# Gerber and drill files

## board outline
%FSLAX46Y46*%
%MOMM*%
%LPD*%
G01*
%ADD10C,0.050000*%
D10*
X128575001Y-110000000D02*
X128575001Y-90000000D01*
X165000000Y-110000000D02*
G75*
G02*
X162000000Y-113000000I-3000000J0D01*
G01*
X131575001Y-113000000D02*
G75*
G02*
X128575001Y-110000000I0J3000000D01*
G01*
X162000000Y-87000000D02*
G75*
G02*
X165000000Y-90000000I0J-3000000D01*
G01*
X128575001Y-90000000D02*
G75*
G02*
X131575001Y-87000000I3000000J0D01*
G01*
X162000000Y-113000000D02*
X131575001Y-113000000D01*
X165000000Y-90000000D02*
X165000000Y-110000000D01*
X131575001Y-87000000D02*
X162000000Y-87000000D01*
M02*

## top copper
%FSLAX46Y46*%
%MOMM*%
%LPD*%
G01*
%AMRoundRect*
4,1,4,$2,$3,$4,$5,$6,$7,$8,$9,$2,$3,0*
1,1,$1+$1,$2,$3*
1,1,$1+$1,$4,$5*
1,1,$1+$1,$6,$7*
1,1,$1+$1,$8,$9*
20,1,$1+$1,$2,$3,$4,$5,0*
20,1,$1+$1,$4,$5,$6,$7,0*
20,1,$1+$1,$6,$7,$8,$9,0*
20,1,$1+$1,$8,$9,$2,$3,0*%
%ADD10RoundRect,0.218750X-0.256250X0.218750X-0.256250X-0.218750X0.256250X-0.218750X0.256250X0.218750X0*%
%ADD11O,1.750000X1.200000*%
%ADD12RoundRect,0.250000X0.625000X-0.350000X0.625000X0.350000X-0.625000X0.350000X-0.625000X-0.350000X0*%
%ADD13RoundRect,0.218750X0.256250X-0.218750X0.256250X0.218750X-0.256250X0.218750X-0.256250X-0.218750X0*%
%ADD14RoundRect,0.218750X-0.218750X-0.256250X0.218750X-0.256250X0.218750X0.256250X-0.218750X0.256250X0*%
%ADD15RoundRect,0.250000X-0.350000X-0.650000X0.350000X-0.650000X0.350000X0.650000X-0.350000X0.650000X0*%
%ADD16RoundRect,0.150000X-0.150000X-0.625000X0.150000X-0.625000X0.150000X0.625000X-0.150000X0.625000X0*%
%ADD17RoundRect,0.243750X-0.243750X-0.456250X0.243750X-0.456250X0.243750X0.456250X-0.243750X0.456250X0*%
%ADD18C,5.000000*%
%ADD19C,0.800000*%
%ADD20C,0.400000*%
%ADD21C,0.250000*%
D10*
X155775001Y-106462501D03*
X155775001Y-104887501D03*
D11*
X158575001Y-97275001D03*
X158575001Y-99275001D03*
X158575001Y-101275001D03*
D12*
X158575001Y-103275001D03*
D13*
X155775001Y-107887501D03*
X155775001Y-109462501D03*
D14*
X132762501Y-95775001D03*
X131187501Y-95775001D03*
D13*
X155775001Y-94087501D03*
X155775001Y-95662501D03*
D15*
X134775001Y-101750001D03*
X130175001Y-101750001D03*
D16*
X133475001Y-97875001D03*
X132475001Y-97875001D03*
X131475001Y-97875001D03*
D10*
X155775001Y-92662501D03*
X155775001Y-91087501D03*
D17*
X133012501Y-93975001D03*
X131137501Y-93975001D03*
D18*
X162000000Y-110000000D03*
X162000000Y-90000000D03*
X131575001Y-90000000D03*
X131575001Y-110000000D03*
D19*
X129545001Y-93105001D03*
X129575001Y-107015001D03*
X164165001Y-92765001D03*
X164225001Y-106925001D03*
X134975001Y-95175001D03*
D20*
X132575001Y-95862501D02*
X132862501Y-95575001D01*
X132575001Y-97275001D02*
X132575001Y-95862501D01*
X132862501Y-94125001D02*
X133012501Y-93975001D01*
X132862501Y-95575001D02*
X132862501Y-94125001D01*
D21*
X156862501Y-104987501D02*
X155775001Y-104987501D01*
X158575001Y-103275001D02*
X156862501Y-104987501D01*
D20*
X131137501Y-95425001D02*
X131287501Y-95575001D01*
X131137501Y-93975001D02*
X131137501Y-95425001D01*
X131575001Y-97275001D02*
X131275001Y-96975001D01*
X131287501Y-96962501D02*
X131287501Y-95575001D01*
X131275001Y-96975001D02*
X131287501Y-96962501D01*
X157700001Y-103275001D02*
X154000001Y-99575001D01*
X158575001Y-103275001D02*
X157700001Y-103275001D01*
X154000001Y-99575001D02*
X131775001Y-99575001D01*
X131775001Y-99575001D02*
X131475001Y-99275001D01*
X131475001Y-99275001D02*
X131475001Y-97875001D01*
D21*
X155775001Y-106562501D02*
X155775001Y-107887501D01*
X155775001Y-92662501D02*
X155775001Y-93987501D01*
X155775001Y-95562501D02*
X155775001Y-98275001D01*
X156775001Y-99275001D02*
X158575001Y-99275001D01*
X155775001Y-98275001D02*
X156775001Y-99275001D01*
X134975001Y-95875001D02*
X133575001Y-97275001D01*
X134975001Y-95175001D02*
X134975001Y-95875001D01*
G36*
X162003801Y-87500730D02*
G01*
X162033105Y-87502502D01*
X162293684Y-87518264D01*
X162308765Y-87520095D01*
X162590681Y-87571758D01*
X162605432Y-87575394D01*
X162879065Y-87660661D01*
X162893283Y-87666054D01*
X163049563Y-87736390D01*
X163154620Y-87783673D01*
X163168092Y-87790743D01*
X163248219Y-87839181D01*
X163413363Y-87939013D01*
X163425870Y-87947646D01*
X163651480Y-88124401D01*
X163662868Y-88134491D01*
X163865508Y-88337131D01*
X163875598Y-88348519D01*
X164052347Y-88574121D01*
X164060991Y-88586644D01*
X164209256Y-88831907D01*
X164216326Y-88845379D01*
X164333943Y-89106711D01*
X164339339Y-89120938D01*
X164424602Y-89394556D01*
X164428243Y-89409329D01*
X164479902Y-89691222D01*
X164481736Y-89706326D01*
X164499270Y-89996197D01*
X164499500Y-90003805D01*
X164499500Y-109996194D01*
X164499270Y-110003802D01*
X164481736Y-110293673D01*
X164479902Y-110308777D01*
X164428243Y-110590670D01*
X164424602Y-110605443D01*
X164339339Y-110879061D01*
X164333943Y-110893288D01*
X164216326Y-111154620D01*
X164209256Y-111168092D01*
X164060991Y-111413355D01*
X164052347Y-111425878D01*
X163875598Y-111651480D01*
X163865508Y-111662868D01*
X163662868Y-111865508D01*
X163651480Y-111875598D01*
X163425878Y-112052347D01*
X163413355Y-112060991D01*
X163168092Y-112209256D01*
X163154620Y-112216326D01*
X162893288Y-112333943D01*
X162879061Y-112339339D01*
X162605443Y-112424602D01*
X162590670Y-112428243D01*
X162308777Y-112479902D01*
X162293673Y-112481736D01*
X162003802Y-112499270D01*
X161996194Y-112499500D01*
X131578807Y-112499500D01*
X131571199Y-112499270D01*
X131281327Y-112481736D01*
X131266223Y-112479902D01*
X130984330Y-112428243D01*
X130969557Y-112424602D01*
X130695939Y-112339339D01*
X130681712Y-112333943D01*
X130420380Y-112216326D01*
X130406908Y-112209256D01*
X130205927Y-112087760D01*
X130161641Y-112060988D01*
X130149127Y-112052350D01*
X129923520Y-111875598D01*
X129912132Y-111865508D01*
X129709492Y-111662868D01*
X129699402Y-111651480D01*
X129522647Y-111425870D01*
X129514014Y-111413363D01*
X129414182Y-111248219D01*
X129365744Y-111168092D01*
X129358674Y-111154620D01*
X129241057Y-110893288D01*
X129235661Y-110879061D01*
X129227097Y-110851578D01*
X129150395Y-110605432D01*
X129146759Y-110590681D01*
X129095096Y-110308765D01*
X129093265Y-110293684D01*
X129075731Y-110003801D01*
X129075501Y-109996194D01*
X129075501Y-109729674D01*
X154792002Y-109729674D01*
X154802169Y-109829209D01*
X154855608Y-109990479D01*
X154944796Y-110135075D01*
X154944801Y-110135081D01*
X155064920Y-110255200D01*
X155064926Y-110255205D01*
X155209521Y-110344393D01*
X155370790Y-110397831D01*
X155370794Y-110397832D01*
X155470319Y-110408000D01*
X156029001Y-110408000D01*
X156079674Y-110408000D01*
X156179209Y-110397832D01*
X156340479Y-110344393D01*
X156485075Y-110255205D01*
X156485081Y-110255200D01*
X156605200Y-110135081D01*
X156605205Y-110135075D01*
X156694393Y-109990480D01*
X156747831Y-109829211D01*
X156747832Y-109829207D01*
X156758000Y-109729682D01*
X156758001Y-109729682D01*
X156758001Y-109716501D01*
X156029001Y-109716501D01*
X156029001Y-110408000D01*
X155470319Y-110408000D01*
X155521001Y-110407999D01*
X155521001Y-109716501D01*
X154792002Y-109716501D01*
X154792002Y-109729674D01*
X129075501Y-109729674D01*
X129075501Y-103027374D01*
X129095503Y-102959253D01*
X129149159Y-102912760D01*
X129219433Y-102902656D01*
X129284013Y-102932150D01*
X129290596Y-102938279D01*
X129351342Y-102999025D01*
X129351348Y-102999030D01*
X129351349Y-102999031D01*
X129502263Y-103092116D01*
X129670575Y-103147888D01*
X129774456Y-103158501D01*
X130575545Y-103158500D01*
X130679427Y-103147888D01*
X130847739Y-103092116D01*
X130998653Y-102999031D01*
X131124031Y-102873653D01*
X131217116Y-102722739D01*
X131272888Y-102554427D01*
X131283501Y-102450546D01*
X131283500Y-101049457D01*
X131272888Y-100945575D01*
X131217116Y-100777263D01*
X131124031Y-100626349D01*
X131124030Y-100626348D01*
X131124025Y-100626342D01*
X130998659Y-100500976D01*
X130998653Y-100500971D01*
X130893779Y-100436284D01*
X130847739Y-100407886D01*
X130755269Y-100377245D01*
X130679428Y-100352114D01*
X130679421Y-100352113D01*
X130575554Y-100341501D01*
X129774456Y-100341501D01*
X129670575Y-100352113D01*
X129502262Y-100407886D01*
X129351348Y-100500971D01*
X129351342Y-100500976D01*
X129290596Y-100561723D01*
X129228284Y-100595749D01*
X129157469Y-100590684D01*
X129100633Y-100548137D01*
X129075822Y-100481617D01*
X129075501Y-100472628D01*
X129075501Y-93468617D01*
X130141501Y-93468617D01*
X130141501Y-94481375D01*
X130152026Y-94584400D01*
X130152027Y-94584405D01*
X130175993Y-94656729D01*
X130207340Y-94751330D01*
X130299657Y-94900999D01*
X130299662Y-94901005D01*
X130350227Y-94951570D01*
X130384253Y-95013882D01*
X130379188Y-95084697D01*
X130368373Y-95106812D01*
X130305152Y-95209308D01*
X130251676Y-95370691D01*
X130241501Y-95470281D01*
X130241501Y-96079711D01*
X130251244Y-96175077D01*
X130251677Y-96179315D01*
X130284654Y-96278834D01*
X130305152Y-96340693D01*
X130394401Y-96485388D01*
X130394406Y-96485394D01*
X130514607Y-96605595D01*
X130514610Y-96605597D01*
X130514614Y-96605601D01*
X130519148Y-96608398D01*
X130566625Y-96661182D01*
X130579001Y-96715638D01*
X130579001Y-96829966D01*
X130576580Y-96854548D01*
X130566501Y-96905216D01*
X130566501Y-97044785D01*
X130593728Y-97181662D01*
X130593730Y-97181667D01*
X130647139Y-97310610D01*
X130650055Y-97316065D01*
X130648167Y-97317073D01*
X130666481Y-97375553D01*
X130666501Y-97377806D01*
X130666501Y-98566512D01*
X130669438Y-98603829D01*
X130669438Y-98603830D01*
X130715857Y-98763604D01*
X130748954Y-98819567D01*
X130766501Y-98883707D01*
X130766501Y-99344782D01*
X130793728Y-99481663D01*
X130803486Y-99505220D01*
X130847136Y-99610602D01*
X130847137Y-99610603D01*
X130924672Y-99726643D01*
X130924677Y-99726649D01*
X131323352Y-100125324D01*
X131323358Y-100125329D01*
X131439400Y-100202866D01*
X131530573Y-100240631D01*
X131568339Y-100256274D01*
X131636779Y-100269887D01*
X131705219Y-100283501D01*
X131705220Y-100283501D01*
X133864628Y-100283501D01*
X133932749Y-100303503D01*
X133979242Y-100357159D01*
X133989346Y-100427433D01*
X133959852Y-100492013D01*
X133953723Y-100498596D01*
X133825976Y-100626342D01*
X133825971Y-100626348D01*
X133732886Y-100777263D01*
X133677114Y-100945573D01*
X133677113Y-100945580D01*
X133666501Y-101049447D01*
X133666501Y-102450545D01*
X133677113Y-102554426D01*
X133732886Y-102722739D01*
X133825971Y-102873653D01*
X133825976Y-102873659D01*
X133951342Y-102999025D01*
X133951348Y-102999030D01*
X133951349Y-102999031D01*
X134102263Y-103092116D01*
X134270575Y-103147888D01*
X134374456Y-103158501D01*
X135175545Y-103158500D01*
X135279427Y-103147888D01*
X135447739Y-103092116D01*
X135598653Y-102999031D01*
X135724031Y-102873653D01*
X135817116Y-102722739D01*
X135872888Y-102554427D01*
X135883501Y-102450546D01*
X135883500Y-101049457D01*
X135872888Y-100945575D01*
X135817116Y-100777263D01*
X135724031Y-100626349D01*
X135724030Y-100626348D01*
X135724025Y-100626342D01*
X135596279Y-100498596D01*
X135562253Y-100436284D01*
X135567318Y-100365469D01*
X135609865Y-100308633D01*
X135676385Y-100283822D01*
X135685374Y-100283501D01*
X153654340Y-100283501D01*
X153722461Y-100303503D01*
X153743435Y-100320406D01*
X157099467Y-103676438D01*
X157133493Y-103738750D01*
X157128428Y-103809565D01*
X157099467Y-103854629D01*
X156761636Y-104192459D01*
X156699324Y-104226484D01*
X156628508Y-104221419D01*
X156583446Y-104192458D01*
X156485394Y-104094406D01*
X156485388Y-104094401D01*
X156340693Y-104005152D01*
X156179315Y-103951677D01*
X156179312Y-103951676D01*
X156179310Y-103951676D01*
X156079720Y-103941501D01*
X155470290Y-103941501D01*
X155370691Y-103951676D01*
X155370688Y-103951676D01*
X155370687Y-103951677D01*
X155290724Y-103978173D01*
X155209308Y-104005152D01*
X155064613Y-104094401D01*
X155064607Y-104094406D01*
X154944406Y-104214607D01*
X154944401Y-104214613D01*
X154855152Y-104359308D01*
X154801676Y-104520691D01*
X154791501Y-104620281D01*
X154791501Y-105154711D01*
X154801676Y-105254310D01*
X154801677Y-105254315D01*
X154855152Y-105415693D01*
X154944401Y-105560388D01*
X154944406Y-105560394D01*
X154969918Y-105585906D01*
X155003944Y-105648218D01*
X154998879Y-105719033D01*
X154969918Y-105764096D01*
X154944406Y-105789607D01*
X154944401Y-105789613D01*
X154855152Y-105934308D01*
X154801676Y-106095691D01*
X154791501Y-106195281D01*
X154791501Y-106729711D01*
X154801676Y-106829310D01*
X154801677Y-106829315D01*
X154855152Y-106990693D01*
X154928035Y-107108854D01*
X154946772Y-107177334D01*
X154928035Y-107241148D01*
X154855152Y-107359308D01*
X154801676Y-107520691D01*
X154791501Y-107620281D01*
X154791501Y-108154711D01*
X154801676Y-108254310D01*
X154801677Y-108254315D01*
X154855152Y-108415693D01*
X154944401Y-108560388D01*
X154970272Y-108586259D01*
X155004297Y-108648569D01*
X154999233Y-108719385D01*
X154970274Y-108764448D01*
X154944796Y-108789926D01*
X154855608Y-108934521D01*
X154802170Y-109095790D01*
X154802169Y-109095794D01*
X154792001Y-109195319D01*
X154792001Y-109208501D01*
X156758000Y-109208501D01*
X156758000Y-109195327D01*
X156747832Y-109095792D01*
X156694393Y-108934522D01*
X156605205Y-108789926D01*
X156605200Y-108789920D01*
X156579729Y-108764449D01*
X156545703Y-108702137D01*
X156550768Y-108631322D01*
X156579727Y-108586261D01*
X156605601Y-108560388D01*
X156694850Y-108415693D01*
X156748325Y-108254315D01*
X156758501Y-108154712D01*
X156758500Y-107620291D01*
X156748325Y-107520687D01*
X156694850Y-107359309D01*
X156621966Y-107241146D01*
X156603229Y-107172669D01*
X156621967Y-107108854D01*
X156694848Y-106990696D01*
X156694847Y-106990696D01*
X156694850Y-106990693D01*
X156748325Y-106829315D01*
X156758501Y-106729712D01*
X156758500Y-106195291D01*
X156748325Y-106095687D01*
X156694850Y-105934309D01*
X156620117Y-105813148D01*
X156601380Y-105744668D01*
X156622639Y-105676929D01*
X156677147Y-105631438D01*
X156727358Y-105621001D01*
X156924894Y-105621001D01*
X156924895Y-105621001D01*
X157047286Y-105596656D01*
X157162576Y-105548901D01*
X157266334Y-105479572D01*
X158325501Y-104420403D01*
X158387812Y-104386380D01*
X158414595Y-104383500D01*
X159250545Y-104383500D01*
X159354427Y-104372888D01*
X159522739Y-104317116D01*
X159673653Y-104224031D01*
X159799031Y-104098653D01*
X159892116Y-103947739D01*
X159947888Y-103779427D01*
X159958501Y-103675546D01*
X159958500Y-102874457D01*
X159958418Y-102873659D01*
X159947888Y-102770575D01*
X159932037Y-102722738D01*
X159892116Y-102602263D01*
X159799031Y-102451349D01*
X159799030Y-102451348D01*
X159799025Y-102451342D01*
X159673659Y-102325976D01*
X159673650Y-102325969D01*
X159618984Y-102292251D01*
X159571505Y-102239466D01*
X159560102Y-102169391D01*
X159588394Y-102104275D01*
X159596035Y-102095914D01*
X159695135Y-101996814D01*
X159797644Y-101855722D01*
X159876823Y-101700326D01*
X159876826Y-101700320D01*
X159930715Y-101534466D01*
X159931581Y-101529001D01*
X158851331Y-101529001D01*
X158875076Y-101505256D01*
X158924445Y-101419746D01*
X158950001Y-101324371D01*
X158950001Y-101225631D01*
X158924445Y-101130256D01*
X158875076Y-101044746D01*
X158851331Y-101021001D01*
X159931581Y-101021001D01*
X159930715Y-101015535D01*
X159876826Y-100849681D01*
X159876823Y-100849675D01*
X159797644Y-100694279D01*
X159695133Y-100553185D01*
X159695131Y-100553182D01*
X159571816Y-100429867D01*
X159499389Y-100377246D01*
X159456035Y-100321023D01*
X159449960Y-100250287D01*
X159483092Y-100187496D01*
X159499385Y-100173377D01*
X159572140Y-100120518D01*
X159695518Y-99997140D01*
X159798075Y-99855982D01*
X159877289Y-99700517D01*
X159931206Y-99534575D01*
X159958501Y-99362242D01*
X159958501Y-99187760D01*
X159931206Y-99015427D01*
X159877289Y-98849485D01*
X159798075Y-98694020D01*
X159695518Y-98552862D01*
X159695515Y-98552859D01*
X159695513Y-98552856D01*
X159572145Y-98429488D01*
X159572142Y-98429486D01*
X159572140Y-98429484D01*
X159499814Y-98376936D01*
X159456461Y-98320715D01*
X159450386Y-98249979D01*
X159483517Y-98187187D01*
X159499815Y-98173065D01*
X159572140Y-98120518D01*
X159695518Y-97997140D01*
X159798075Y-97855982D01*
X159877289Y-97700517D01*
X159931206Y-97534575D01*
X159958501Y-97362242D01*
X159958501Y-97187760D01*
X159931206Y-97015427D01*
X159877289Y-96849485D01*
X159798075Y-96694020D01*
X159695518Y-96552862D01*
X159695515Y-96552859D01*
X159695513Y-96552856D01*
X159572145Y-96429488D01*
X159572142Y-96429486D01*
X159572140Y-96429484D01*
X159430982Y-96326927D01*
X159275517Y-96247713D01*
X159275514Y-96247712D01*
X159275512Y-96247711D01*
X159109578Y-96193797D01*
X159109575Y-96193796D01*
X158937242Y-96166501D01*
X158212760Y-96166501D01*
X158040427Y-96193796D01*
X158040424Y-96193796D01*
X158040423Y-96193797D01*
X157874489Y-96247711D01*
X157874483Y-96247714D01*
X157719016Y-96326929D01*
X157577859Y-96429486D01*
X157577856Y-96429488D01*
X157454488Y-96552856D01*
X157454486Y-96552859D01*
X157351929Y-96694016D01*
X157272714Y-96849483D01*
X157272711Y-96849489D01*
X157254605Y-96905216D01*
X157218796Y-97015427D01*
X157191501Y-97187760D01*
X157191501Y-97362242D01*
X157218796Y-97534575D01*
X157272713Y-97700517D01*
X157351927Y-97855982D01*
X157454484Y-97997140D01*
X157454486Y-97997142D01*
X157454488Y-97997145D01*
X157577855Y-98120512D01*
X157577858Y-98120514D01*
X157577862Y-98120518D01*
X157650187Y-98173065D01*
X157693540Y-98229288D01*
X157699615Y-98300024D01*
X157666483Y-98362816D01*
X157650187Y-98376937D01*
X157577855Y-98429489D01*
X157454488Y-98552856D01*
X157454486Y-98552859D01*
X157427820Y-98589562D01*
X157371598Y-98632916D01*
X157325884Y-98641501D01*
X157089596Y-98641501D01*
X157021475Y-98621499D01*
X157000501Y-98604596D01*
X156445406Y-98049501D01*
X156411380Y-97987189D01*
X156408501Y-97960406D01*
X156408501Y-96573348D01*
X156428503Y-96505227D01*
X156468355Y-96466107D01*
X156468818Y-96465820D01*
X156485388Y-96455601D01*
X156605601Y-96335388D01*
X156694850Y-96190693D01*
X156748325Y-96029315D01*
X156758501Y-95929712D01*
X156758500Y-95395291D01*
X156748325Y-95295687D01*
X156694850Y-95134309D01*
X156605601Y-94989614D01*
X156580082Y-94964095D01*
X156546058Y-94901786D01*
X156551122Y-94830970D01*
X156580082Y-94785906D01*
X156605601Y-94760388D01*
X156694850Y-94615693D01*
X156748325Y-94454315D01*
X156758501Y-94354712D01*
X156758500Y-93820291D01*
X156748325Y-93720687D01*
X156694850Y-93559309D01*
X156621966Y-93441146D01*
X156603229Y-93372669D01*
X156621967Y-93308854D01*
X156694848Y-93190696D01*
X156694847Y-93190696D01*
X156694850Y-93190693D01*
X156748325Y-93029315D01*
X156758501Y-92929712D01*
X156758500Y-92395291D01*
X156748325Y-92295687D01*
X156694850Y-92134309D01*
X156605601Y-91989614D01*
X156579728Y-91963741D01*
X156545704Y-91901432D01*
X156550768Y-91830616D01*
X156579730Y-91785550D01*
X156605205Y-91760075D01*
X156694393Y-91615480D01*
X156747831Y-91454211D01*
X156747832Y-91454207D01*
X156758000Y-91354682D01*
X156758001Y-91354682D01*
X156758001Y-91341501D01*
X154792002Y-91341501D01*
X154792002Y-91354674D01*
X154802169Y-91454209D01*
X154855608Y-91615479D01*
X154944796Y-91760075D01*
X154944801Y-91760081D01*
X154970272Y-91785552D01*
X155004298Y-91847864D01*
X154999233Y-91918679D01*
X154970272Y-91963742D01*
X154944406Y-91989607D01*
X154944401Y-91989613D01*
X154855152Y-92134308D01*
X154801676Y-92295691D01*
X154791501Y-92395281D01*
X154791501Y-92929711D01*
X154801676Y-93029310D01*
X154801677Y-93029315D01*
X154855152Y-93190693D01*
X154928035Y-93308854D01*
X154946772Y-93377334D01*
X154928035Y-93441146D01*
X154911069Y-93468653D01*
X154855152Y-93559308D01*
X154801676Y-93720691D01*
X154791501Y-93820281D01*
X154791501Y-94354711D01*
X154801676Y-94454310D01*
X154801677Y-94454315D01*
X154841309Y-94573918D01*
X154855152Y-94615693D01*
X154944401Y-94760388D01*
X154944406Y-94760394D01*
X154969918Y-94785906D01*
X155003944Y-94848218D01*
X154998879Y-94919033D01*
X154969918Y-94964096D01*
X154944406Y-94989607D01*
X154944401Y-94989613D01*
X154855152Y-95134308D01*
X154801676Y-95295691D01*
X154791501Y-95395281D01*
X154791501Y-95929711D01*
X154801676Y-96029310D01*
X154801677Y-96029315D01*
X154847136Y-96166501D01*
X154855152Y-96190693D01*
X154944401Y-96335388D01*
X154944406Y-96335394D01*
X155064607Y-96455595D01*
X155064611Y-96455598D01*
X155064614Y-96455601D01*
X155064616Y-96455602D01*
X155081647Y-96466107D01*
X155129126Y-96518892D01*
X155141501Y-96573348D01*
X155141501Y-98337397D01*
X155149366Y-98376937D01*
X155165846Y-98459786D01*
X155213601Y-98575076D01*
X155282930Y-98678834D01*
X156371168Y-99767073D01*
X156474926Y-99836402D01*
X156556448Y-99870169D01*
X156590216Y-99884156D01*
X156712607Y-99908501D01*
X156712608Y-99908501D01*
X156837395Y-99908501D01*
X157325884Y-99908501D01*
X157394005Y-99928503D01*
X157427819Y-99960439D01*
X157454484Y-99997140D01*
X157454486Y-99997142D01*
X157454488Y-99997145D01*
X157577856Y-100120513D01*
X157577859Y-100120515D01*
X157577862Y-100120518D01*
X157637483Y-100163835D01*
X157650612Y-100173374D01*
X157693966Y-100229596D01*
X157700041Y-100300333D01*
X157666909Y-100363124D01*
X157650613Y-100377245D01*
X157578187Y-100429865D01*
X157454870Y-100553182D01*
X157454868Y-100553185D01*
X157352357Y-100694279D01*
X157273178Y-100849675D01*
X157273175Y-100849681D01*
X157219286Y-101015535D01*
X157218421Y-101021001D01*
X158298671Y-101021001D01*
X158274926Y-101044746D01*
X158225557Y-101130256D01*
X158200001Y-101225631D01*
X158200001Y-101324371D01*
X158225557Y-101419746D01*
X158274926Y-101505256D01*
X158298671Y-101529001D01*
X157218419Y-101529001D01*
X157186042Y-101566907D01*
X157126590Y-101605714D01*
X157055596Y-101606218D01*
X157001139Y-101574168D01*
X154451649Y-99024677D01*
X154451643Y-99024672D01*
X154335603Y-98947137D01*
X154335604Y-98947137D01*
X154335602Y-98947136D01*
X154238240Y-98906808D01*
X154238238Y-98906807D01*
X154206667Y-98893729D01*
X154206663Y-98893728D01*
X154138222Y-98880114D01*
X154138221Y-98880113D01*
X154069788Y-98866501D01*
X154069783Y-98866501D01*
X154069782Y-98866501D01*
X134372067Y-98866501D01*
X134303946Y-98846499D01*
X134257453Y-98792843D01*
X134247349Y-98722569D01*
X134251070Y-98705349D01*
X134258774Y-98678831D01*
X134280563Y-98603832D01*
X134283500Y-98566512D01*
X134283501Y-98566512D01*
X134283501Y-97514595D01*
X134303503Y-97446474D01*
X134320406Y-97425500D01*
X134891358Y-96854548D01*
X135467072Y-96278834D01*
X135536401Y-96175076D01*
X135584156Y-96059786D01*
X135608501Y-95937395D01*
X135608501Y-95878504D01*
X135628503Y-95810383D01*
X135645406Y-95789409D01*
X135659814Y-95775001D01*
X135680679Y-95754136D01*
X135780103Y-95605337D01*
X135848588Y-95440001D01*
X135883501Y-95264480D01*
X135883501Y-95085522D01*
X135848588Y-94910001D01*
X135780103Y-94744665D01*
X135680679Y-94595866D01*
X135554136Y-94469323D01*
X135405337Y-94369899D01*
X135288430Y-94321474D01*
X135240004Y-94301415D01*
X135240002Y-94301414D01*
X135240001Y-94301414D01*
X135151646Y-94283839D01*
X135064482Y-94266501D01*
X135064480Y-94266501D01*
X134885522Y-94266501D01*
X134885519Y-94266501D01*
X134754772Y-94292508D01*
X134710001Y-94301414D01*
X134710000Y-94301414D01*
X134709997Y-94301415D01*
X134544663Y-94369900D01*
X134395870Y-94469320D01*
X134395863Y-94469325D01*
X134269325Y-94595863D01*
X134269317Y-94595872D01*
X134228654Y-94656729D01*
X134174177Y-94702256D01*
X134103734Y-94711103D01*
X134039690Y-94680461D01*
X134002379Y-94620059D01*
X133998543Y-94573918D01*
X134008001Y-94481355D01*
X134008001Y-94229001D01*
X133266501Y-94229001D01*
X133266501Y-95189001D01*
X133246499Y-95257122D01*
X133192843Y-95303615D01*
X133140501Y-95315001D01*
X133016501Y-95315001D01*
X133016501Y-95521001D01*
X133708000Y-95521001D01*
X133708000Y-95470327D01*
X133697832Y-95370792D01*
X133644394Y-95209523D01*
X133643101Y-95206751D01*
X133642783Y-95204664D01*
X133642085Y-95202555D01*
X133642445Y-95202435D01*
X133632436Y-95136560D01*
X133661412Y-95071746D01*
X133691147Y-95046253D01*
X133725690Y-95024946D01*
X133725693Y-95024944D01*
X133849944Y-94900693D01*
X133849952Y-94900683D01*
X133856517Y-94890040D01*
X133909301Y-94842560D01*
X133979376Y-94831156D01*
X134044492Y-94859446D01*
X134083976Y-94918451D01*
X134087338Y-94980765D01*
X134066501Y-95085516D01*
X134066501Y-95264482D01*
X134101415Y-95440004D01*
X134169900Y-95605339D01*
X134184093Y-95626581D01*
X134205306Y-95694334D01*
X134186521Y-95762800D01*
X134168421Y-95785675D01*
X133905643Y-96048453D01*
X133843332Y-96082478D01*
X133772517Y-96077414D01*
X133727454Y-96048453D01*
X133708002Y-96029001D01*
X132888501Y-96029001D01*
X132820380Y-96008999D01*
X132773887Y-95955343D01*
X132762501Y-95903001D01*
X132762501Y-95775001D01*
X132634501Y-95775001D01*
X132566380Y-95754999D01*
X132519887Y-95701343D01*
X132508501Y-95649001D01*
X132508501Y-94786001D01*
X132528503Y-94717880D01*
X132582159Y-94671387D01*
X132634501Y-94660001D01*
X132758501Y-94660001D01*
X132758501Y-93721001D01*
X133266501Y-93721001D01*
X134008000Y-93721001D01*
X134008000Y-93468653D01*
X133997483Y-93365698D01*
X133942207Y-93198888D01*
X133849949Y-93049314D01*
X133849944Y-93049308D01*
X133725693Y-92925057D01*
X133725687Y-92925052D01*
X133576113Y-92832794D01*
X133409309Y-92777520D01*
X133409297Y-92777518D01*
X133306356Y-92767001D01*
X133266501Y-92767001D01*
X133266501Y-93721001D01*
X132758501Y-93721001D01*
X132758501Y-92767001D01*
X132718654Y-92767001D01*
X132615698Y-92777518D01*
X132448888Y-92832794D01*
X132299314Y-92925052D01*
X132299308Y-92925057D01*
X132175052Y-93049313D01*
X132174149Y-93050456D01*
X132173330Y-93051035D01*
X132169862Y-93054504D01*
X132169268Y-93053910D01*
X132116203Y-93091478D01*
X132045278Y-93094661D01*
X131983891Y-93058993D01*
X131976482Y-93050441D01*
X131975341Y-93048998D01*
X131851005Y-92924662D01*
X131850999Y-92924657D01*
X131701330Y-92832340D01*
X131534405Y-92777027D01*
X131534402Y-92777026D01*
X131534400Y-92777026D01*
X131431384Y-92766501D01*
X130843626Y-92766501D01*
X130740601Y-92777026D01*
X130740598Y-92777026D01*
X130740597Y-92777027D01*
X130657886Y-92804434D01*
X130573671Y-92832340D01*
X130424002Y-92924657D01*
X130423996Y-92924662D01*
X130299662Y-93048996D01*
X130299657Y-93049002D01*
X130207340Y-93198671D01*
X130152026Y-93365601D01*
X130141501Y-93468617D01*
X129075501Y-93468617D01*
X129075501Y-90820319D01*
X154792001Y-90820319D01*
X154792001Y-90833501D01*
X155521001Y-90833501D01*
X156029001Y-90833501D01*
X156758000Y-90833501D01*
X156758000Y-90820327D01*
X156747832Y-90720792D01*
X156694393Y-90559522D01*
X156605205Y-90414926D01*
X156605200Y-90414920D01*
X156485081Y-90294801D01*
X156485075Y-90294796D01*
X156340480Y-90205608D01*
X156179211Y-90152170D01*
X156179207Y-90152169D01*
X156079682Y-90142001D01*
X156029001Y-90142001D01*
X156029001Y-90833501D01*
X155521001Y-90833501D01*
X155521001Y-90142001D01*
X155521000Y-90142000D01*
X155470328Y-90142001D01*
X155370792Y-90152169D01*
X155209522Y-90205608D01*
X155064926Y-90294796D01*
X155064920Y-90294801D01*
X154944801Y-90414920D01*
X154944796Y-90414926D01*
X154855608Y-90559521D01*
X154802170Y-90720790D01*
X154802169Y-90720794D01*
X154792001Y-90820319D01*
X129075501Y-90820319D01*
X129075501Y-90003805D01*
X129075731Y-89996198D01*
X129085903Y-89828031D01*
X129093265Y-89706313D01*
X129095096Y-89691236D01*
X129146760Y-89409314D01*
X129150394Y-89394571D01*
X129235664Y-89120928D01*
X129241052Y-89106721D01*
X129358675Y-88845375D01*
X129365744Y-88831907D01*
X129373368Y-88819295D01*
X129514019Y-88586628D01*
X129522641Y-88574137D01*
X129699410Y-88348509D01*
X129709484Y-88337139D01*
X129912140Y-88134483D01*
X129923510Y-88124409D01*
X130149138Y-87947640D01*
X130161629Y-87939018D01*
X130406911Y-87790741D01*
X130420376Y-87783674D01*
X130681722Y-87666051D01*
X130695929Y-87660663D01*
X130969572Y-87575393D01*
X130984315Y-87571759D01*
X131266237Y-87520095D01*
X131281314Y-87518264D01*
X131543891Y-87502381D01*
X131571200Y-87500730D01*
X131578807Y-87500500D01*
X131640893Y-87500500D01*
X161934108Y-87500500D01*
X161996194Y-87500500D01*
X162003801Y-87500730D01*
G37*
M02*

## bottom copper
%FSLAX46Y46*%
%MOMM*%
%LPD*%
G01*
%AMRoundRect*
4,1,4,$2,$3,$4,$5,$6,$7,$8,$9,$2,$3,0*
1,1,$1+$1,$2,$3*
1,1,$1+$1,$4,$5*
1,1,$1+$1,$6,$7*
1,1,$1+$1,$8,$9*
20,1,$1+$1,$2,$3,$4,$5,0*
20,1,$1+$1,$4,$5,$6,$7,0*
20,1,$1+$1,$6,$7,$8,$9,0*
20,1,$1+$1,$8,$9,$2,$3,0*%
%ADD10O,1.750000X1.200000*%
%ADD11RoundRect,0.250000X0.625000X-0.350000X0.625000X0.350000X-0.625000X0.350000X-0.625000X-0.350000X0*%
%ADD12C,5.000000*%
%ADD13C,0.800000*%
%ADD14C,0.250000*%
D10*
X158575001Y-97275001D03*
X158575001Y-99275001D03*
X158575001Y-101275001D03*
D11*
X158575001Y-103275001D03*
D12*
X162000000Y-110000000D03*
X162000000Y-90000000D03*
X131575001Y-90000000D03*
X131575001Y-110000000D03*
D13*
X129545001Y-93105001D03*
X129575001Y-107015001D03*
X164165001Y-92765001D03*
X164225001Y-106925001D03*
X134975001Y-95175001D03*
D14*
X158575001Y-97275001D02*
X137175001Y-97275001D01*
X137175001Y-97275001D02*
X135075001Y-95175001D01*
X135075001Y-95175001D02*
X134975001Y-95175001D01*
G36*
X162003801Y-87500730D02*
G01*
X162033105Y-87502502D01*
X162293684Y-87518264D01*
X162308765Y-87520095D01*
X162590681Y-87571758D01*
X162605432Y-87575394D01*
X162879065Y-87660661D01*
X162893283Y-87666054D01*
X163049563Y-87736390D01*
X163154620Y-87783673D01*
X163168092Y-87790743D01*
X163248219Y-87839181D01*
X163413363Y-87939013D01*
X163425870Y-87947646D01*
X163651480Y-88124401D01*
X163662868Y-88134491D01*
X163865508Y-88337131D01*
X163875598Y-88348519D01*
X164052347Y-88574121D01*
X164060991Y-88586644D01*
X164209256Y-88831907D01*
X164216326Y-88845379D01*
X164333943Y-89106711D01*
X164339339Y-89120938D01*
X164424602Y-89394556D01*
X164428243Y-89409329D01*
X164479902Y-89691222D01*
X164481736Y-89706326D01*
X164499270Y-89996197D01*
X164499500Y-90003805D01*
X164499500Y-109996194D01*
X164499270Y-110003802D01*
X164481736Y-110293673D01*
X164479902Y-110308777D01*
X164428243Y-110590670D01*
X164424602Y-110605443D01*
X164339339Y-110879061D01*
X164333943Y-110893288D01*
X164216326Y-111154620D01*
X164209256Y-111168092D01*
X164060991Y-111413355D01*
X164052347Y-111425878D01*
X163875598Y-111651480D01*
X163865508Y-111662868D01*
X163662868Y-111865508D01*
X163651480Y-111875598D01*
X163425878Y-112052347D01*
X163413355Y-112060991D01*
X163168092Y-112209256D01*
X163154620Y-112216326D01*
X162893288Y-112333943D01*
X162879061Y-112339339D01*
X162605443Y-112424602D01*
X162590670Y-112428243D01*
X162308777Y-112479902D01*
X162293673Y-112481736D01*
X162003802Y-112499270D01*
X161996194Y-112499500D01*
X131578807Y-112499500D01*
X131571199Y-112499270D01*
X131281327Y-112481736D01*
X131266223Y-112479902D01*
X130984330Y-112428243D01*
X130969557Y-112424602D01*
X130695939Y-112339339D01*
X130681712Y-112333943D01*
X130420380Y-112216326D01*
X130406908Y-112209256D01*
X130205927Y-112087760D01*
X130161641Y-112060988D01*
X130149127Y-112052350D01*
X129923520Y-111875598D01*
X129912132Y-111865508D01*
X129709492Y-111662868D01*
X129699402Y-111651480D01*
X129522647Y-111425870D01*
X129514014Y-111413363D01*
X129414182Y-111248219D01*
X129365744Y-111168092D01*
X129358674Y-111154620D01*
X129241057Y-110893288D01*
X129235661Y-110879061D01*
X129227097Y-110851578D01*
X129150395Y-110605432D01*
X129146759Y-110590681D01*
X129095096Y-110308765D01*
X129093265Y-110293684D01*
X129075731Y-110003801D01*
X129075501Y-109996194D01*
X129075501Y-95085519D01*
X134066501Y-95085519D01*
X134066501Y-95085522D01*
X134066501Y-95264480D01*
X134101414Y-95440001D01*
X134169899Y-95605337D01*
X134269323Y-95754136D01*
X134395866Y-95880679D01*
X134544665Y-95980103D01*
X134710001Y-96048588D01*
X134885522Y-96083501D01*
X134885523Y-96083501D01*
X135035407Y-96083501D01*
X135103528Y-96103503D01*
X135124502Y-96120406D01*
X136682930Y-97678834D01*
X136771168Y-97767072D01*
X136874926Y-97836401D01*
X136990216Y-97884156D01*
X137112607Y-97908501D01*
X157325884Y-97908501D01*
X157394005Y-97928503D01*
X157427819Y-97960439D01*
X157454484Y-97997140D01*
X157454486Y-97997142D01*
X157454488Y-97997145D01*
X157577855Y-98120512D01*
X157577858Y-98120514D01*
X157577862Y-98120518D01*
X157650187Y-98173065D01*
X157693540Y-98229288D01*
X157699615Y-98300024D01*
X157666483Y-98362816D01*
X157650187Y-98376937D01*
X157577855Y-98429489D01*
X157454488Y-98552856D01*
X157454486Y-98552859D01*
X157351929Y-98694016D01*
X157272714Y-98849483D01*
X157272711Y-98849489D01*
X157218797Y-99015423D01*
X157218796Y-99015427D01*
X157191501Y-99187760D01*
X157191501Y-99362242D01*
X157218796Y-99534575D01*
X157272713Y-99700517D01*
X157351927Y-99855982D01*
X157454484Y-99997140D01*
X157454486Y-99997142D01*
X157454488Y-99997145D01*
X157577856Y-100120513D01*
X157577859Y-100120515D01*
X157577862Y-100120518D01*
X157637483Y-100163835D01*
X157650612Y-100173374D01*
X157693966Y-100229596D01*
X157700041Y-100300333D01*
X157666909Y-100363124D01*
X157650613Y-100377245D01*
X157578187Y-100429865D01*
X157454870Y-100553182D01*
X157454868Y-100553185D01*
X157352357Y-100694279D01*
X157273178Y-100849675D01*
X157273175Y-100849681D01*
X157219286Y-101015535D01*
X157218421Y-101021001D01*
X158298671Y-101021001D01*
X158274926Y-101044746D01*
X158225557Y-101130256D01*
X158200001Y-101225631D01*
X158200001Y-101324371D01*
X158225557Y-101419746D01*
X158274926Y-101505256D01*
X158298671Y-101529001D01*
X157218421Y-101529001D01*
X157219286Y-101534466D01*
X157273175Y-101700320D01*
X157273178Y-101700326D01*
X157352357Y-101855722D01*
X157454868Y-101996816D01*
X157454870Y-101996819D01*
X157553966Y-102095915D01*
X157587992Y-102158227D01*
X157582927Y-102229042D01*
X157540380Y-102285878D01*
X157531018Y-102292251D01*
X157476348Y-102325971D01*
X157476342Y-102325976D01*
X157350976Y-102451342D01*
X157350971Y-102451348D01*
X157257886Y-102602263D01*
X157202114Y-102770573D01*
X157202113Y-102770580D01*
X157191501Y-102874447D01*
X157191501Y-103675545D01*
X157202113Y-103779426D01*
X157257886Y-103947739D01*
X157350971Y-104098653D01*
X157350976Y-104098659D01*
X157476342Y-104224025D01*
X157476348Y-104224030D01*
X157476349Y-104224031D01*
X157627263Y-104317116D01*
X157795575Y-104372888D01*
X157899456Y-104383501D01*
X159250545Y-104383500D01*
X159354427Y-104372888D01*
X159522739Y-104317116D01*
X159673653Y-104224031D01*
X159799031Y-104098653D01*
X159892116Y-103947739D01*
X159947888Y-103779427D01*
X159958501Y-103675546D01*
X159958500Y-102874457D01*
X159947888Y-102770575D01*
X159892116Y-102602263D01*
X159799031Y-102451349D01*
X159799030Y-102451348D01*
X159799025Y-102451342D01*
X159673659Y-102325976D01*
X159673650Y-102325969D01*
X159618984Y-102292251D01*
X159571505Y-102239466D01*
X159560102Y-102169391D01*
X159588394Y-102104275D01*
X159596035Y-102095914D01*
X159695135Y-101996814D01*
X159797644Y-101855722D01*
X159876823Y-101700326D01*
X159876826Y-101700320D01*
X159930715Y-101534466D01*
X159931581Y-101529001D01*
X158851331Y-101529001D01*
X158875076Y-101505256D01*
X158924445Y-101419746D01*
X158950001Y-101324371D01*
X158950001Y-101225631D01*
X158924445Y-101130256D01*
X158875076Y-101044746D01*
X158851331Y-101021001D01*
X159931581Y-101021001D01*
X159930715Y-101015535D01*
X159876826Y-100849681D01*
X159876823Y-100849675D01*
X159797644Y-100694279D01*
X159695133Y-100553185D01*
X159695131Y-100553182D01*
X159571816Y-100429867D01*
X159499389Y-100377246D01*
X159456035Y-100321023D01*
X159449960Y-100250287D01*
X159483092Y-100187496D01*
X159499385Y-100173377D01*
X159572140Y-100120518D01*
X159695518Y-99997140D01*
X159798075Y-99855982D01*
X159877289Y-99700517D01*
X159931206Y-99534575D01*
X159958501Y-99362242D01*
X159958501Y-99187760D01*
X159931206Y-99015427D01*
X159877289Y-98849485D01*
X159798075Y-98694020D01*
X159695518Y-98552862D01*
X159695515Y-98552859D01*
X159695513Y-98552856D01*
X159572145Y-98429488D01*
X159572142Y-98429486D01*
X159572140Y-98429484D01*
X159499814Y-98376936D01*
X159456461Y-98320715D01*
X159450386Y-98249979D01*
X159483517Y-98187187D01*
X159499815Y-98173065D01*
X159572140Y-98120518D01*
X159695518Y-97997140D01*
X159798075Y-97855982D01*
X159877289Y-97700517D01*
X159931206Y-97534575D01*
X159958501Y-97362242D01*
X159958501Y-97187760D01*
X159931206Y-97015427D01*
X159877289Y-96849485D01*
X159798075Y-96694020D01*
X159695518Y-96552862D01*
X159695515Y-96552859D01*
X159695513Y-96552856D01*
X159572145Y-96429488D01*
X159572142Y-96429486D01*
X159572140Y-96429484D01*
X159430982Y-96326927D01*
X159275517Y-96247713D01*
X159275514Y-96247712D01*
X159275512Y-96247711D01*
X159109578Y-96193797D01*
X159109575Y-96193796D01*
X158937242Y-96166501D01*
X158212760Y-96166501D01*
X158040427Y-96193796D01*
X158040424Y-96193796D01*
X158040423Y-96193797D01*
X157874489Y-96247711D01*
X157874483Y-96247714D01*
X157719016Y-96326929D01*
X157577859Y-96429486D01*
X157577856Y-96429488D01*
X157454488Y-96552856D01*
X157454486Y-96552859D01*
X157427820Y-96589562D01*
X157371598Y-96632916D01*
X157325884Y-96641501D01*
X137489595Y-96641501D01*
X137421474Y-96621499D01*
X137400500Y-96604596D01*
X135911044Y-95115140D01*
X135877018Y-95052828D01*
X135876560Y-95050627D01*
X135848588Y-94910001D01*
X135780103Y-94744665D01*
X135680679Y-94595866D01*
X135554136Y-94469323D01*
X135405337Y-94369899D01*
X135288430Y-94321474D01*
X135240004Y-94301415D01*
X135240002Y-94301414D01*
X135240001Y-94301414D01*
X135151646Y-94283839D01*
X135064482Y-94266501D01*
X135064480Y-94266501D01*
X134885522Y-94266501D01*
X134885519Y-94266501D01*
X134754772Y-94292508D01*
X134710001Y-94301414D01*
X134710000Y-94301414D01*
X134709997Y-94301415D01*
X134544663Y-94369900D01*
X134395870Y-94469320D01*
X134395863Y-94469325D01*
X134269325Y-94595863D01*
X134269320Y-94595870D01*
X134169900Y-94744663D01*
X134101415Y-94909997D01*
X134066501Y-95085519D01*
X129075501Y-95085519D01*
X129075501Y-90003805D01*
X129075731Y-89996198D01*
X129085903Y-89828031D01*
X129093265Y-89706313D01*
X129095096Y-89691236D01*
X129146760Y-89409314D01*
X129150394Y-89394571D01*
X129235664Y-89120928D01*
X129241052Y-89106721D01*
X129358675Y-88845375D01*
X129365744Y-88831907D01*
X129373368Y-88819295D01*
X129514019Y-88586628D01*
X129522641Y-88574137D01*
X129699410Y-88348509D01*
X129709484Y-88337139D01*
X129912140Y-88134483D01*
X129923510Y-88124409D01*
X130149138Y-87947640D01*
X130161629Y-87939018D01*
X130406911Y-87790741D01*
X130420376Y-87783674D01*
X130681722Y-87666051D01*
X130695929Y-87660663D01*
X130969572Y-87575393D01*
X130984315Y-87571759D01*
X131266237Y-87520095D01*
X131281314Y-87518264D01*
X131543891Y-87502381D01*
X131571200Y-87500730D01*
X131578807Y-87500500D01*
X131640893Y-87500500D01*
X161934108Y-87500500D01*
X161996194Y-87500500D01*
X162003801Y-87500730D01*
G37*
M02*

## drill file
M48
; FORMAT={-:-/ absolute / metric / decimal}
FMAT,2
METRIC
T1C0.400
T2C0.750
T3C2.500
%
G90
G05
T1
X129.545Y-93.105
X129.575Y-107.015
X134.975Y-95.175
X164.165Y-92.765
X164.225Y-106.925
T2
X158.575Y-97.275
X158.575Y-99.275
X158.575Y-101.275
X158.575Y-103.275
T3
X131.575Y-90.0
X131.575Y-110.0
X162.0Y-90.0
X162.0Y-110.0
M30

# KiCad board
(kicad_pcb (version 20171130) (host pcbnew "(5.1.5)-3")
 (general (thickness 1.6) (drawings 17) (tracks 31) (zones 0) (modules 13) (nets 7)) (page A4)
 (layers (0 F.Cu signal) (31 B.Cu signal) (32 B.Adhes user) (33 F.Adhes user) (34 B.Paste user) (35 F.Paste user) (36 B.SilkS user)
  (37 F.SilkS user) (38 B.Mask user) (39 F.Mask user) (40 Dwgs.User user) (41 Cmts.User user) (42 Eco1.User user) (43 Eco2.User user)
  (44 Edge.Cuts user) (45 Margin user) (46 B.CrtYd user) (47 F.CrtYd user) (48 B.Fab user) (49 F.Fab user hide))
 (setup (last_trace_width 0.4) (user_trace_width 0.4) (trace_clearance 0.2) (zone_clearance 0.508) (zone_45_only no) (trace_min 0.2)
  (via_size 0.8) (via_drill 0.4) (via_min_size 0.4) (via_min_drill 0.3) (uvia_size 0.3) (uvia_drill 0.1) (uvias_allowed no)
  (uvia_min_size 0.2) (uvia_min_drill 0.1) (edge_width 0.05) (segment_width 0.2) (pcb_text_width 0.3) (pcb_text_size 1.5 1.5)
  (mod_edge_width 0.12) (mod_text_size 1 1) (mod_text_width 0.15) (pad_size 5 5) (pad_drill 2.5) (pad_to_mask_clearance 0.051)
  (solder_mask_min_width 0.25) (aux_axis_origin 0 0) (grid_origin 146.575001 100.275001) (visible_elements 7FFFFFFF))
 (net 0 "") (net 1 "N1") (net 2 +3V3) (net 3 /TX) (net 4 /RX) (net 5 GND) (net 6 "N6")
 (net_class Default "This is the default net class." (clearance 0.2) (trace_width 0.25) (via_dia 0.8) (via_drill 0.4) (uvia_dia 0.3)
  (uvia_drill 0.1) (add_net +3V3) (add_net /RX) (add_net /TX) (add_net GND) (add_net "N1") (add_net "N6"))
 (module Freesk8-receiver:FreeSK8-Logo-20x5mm (layer B.Cu) (at 146.375001 100.375001 180)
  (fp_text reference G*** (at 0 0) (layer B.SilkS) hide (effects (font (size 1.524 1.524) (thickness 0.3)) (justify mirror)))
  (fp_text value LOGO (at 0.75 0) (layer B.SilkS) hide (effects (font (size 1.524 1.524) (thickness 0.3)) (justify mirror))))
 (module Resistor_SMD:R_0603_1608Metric (layer F.Cu) (at 155.775001 105.675001 270)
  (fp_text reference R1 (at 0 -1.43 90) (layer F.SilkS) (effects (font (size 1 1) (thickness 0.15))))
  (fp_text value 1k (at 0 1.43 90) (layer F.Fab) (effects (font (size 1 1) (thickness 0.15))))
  (pad 2 smd roundrect (at 0.7875 0 270) (size 0.875 0.95) (layers F.Cu F.Paste F.Mask) (roundrect_rratio 0.25) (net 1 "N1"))
  (pad 1 smd roundrect (at -0.7875 0 270) (size 0.875 0.95) (layers F.Cu F.Paste F.Mask) (roundrect_rratio 0.25) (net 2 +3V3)))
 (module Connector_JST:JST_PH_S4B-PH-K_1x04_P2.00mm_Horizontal (layer F.Cu) (at 158.575001 103.275001 90)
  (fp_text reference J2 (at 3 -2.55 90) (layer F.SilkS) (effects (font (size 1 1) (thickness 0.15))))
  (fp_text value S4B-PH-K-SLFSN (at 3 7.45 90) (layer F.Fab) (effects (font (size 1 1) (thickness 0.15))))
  (pad 4 thru_hole oval (at 6 0 90) (size 1.2 1.75) (drill 0.75) (layers *.Cu *.Mask) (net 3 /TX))
  (pad 3 thru_hole oval (at 4 0 90) (size 1.2 1.75) (drill 0.75) (layers *.Cu *.Mask) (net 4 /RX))
  (pad 2 thru_hole oval (at 2 0 90) (size 1.2 1.75) (drill 0.75) (layers *.Cu *.Mask) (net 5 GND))
  (pad 1 thru_hole roundrect (at 0 0 90) (size 1.2 1.75) (drill 0.75) (layers *.Cu *.Mask) (roundrect_rratio 0.208333) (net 2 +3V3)))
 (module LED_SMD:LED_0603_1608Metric (layer F.Cu) (at 155.775001 108.675001 90)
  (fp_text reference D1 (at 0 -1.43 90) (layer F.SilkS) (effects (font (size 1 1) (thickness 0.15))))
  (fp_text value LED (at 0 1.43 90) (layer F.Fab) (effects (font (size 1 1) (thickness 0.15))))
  (pad 2 smd roundrect (at 0.7875 0 90) (size 0.875 0.95) (layers F.Cu F.Paste F.Mask) (roundrect_rratio 0.25) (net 1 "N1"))
  (pad 1 smd roundrect (at -0.7875 0 90) (size 0.875 0.95) (layers F.Cu F.Paste F.Mask) (roundrect_rratio 0.25) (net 5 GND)))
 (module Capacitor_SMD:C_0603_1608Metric (layer F.Cu) (at 131.975001 95.775001)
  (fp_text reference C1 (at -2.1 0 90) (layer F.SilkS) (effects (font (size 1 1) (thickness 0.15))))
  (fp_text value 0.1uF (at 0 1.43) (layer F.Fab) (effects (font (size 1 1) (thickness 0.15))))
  (pad 2 smd roundrect (at 0.7875 0) (size 0.875 0.95) (layers F.Cu F.Paste F.Mask) (roundrect_rratio 0.25) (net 5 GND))
  (pad 1 smd roundrect (at -0.7875 0) (size 0.875 0.95) (layers F.Cu F.Paste F.Mask) (roundrect_rratio 0.25) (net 2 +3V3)))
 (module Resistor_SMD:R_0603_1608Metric (layer F.Cu) (at 155.775001 94.875001 90)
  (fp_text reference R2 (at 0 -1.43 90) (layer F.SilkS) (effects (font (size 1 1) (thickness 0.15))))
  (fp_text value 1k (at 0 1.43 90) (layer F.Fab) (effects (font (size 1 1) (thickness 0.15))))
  (pad 2 smd roundrect (at 0.7875 0 90) (size 0.875 0.95) (layers F.Cu F.Paste F.Mask) (roundrect_rratio 0.25) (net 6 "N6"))
  (pad 1 smd roundrect (at -0.7875 0 90) (size 0.875 0.95) (layers F.Cu F.Paste F.Mask) (roundrect_rratio 0.25) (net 4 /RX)))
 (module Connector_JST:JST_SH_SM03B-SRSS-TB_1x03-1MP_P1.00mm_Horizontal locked (layer F.Cu) (at 132.475001 99.875001)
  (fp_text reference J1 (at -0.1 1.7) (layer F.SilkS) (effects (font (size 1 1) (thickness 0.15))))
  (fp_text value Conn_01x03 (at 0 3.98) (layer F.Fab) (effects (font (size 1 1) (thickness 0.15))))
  (pad MP smd roundrect (at 2.3 1.875) (size 1.2 1.8) (layers F.Cu F.Paste F.Mask) (roundrect_rratio 0.208333))
  (pad MP smd roundrect (at -2.3 1.875) (size 1.2 1.8) (layers F.Cu F.Paste F.Mask) (roundrect_rratio 0.208333))
  (pad 3 smd roundrect (at 1 -2) (size 0.6 1.55) (layers F.Cu F.Paste F.Mask) (roundrect_rratio 0.25) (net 3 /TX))
  (pad 2 smd roundrect (at 0 -2) (size 0.6 1.55) (layers F.Cu F.Paste F.Mask) (roundrect_rratio 0.25) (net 5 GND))
  (pad 1 smd roundrect (at -1 -2) (size 0.6 1.55) (layers F.Cu F.Paste F.Mask) (roundrect_rratio 0.25) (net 2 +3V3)))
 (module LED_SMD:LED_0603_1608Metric (layer F.Cu) (at 155.775001 91.875001 270)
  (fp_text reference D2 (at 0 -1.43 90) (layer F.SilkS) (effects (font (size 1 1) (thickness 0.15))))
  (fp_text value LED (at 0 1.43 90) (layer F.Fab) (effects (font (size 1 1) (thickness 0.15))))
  (pad 2 smd roundrect (at 0.7875 0 270) (size 0.875 0.95) (layers F.Cu F.Paste F.Mask) (roundrect_rratio 0.25) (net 6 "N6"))
  (pad 1 smd roundrect (at -0.7875 0 270) (size 0.875 0.95) (layers F.Cu F.Paste F.Mask) (roundrect_rratio 0.25) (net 5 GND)))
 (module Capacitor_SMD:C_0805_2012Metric (layer F.Cu) (at 132.075001 93.975001)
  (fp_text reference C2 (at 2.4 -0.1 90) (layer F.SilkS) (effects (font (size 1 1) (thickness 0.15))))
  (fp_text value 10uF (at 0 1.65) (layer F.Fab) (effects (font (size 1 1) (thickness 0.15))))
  (pad 2 smd roundrect (at 0.9375 0) (size 0.975 1.4) (layers F.Cu F.Paste F.Mask) (roundrect_rratio 0.25) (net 5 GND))
  (pad 1 smd roundrect (at -0.9375 0) (size 0.975 1.4) (layers F.Cu F.Paste F.Mask) (roundrect_rratio 0.25) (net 2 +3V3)))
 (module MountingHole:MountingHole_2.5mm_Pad (layer F.Cu) (at 162 110) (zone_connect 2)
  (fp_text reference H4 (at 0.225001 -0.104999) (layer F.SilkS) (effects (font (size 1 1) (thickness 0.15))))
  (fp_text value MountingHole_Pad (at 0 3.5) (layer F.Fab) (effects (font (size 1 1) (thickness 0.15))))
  (pad 1 thru_hole circle (at 0 0) (size 5 5) (drill 2.5) (layers *.Cu *.Mask) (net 5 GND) (zone_connect 2)))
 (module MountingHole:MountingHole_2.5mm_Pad (layer F.Cu) (at 162 90) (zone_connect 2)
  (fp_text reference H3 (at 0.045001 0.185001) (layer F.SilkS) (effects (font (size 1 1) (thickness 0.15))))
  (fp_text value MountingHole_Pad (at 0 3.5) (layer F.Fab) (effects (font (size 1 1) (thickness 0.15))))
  (pad 1 thru_hole circle (at 0 0) (size 5 5) (drill 2.5) (layers *.Cu *.Mask) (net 5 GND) (zone_connect 2)))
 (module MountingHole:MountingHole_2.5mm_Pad (layer F.Cu) (at 131.575001 90) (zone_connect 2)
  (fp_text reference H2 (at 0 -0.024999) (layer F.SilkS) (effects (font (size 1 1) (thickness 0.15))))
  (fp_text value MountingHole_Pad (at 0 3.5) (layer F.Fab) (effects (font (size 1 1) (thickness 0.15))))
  (pad 1 thru_hole circle (at 0 0) (size 5 5) (drill 2.5) (layers *.Cu *.Mask) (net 5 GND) (zone_connect 2)))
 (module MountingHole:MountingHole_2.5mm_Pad (layer F.Cu) (at 131.575001 110) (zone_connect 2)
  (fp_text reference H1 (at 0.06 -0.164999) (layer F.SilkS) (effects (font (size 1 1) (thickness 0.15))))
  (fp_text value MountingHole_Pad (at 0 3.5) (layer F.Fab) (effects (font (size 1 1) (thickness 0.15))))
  (pad 1 thru_hole circle (at 0 0) (size 5 5) (drill 2.5) (layers *.Cu *.Mask) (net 5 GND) (zone_connect 2)))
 (gr_line (start 128.575001 110) (end 128.575001 90) (layer Edge.Cuts) (width 0.05))
 (gr_arc (start 162 110) (end 162 113) (angle -90) (layer Edge.Cuts) (width 0.05))
 (gr_arc (start 131.575001 110) (end 128.575001 110) (angle -90) (layer Edge.Cuts) (width 0.05))
 (gr_arc (start 162 90) (end 165 90) (angle -90) (layer Edge.Cuts) (width 0.05))
 (gr_arc (start 131.575001 90) (end 131.575001 87) (angle -90) (layer Edge.Cuts) (width 0.05))
 (gr_line (start 162 113) (end 131.575001 113) (layer Edge.Cuts) (width 0.05))
 (gr_line (start 165 90) (end 165 110) (layer Edge.Cuts) (width 0.05))
 (gr_line (start 131.575001 87) (end 162 87) (layer Edge.Cuts) (width 0.05))
 (via (at 129.545001 93.105001) (size 0.8) (drill 0.4) (layers F.Cu B.Cu) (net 5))
 (via (at 129.575001 107.015001) (size 0.8) (drill 0.4) (layers F.Cu B.Cu) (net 5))
 (via (at 164.165001 92.765001) (size 0.8) (drill 0.4) (layers F.Cu B.Cu) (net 5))
 (via (at 164.225001 106.925001) (size 0.8) (drill 0.4) (layers F.Cu B.Cu) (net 5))
 (segment (start 132.575001 95.862501) (end 132.862501 95.575001) (width 0.4) (layer F.Cu) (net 5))
 (segment (start 132.575001 97.275001) (end 132.575001 95.862501) (width 0.4) (layer F.Cu) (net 5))
 (segment (start 132.862501 94.125001) (end 133.012501 93.975001) (width 0.4) (layer F.Cu) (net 5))
 (segment (start 132.862501 95.575001) (end 132.862501 94.125001) (width 0.4) (layer F.Cu) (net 5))
 (segment (start 156.862501 104.987501) (end 155.775001 104.987501) (width 0.25) (layer F.Cu) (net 2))
 (segment (start 158.575001 103.275001) (end 156.862501 104.987501) (width 0.25) (layer F.Cu) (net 2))
 (segment (start 131.137501 95.425001) (end 131.287501 95.575001) (width 0.4) (layer F.Cu) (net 2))
 (segment (start 131.137501 93.975001) (end 131.137501 95.425001) (width 0.4) (layer F.Cu) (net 2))
 (segment (start 131.575001 97.275001) (end 131.275001 96.975001) (width 0.4) (layer F.Cu) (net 2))
 (segment (start 131.287501 96.962501) (end 131.287501 95.575001) (width 0.4) (layer F.Cu) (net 2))
 (segment (start 131.275001 96.975001) (end 131.287501 96.962501) (width 0.4) (layer F.Cu) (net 2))
 (segment (start 157.700001 103.275001) (end 154.000001 99.575001) (width 0.4) (layer F.Cu) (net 2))
 (segment (start 158.575001 103.275001) (end 157.700001 103.275001) (width 0.4) (layer F.Cu) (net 2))
 (segment (start 154.000001 99.575001) (end 131.775001 99.575001) (width 0.4) (layer F.Cu) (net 2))
 (segment (start 131.775001 99.575001) (end 131.475001 99.275001) (width 0.4) (layer F.Cu) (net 2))
 (segment (start 131.475001 99.275001) (end 131.475001 97.875001) (width 0.4) (layer F.Cu) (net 2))
 (segment (start 155.775001 106.562501) (end 155.775001 107.887501) (width 0.25) (layer F.Cu) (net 1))
 (segment (start 155.775001 92.662501) (end 155.775001 93.987501) (width 0.25) (layer F.Cu) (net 6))
 (segment (start 155.775001 95.562501) (end 155.775001 98.275001) (width 0.25) (layer F.Cu) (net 4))
 (segment (start 156.775001 99.275001) (end 158.575001 99.275001) (width 0.25) (layer F.Cu) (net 4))
 (segment (start 155.775001 98.275001) (end 156.775001 99.275001) (width 0.25) (layer F.Cu) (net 4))
 (segment (start 158.575001 97.275001) (end 137.175001 97.275001) (width 0.25) (layer B.Cu) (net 3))
 (via (at 134.975001 95.175001) (size 0.8) (drill 0.4) (layers F.Cu B.Cu) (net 3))
 (segment (start 137.175001 97.275001) (end 135.075001 95.175001) (width 0.25) (layer B.Cu) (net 3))
 (segment (start 135.075001 95.175001) (end 134.975001 95.175001) (width 0.25) (layer B.Cu) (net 3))
 (segment (start 134.975001 95.875001) (end 133.575001 97.275001) (width 0.25) (layer F.Cu) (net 3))
 (segment (start 134.975001 95.175001) (end 134.975001 95.875001) (width 0.25) (layer F.Cu) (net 3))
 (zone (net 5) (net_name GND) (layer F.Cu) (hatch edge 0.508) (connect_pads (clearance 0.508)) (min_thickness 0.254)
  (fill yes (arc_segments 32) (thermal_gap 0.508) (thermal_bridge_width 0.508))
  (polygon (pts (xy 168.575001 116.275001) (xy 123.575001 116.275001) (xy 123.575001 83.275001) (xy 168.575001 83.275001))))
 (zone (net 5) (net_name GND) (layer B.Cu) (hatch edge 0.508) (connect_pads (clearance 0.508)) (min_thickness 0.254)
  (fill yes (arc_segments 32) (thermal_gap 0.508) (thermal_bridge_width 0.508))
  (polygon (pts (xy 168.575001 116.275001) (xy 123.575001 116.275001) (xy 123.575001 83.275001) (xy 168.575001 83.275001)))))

